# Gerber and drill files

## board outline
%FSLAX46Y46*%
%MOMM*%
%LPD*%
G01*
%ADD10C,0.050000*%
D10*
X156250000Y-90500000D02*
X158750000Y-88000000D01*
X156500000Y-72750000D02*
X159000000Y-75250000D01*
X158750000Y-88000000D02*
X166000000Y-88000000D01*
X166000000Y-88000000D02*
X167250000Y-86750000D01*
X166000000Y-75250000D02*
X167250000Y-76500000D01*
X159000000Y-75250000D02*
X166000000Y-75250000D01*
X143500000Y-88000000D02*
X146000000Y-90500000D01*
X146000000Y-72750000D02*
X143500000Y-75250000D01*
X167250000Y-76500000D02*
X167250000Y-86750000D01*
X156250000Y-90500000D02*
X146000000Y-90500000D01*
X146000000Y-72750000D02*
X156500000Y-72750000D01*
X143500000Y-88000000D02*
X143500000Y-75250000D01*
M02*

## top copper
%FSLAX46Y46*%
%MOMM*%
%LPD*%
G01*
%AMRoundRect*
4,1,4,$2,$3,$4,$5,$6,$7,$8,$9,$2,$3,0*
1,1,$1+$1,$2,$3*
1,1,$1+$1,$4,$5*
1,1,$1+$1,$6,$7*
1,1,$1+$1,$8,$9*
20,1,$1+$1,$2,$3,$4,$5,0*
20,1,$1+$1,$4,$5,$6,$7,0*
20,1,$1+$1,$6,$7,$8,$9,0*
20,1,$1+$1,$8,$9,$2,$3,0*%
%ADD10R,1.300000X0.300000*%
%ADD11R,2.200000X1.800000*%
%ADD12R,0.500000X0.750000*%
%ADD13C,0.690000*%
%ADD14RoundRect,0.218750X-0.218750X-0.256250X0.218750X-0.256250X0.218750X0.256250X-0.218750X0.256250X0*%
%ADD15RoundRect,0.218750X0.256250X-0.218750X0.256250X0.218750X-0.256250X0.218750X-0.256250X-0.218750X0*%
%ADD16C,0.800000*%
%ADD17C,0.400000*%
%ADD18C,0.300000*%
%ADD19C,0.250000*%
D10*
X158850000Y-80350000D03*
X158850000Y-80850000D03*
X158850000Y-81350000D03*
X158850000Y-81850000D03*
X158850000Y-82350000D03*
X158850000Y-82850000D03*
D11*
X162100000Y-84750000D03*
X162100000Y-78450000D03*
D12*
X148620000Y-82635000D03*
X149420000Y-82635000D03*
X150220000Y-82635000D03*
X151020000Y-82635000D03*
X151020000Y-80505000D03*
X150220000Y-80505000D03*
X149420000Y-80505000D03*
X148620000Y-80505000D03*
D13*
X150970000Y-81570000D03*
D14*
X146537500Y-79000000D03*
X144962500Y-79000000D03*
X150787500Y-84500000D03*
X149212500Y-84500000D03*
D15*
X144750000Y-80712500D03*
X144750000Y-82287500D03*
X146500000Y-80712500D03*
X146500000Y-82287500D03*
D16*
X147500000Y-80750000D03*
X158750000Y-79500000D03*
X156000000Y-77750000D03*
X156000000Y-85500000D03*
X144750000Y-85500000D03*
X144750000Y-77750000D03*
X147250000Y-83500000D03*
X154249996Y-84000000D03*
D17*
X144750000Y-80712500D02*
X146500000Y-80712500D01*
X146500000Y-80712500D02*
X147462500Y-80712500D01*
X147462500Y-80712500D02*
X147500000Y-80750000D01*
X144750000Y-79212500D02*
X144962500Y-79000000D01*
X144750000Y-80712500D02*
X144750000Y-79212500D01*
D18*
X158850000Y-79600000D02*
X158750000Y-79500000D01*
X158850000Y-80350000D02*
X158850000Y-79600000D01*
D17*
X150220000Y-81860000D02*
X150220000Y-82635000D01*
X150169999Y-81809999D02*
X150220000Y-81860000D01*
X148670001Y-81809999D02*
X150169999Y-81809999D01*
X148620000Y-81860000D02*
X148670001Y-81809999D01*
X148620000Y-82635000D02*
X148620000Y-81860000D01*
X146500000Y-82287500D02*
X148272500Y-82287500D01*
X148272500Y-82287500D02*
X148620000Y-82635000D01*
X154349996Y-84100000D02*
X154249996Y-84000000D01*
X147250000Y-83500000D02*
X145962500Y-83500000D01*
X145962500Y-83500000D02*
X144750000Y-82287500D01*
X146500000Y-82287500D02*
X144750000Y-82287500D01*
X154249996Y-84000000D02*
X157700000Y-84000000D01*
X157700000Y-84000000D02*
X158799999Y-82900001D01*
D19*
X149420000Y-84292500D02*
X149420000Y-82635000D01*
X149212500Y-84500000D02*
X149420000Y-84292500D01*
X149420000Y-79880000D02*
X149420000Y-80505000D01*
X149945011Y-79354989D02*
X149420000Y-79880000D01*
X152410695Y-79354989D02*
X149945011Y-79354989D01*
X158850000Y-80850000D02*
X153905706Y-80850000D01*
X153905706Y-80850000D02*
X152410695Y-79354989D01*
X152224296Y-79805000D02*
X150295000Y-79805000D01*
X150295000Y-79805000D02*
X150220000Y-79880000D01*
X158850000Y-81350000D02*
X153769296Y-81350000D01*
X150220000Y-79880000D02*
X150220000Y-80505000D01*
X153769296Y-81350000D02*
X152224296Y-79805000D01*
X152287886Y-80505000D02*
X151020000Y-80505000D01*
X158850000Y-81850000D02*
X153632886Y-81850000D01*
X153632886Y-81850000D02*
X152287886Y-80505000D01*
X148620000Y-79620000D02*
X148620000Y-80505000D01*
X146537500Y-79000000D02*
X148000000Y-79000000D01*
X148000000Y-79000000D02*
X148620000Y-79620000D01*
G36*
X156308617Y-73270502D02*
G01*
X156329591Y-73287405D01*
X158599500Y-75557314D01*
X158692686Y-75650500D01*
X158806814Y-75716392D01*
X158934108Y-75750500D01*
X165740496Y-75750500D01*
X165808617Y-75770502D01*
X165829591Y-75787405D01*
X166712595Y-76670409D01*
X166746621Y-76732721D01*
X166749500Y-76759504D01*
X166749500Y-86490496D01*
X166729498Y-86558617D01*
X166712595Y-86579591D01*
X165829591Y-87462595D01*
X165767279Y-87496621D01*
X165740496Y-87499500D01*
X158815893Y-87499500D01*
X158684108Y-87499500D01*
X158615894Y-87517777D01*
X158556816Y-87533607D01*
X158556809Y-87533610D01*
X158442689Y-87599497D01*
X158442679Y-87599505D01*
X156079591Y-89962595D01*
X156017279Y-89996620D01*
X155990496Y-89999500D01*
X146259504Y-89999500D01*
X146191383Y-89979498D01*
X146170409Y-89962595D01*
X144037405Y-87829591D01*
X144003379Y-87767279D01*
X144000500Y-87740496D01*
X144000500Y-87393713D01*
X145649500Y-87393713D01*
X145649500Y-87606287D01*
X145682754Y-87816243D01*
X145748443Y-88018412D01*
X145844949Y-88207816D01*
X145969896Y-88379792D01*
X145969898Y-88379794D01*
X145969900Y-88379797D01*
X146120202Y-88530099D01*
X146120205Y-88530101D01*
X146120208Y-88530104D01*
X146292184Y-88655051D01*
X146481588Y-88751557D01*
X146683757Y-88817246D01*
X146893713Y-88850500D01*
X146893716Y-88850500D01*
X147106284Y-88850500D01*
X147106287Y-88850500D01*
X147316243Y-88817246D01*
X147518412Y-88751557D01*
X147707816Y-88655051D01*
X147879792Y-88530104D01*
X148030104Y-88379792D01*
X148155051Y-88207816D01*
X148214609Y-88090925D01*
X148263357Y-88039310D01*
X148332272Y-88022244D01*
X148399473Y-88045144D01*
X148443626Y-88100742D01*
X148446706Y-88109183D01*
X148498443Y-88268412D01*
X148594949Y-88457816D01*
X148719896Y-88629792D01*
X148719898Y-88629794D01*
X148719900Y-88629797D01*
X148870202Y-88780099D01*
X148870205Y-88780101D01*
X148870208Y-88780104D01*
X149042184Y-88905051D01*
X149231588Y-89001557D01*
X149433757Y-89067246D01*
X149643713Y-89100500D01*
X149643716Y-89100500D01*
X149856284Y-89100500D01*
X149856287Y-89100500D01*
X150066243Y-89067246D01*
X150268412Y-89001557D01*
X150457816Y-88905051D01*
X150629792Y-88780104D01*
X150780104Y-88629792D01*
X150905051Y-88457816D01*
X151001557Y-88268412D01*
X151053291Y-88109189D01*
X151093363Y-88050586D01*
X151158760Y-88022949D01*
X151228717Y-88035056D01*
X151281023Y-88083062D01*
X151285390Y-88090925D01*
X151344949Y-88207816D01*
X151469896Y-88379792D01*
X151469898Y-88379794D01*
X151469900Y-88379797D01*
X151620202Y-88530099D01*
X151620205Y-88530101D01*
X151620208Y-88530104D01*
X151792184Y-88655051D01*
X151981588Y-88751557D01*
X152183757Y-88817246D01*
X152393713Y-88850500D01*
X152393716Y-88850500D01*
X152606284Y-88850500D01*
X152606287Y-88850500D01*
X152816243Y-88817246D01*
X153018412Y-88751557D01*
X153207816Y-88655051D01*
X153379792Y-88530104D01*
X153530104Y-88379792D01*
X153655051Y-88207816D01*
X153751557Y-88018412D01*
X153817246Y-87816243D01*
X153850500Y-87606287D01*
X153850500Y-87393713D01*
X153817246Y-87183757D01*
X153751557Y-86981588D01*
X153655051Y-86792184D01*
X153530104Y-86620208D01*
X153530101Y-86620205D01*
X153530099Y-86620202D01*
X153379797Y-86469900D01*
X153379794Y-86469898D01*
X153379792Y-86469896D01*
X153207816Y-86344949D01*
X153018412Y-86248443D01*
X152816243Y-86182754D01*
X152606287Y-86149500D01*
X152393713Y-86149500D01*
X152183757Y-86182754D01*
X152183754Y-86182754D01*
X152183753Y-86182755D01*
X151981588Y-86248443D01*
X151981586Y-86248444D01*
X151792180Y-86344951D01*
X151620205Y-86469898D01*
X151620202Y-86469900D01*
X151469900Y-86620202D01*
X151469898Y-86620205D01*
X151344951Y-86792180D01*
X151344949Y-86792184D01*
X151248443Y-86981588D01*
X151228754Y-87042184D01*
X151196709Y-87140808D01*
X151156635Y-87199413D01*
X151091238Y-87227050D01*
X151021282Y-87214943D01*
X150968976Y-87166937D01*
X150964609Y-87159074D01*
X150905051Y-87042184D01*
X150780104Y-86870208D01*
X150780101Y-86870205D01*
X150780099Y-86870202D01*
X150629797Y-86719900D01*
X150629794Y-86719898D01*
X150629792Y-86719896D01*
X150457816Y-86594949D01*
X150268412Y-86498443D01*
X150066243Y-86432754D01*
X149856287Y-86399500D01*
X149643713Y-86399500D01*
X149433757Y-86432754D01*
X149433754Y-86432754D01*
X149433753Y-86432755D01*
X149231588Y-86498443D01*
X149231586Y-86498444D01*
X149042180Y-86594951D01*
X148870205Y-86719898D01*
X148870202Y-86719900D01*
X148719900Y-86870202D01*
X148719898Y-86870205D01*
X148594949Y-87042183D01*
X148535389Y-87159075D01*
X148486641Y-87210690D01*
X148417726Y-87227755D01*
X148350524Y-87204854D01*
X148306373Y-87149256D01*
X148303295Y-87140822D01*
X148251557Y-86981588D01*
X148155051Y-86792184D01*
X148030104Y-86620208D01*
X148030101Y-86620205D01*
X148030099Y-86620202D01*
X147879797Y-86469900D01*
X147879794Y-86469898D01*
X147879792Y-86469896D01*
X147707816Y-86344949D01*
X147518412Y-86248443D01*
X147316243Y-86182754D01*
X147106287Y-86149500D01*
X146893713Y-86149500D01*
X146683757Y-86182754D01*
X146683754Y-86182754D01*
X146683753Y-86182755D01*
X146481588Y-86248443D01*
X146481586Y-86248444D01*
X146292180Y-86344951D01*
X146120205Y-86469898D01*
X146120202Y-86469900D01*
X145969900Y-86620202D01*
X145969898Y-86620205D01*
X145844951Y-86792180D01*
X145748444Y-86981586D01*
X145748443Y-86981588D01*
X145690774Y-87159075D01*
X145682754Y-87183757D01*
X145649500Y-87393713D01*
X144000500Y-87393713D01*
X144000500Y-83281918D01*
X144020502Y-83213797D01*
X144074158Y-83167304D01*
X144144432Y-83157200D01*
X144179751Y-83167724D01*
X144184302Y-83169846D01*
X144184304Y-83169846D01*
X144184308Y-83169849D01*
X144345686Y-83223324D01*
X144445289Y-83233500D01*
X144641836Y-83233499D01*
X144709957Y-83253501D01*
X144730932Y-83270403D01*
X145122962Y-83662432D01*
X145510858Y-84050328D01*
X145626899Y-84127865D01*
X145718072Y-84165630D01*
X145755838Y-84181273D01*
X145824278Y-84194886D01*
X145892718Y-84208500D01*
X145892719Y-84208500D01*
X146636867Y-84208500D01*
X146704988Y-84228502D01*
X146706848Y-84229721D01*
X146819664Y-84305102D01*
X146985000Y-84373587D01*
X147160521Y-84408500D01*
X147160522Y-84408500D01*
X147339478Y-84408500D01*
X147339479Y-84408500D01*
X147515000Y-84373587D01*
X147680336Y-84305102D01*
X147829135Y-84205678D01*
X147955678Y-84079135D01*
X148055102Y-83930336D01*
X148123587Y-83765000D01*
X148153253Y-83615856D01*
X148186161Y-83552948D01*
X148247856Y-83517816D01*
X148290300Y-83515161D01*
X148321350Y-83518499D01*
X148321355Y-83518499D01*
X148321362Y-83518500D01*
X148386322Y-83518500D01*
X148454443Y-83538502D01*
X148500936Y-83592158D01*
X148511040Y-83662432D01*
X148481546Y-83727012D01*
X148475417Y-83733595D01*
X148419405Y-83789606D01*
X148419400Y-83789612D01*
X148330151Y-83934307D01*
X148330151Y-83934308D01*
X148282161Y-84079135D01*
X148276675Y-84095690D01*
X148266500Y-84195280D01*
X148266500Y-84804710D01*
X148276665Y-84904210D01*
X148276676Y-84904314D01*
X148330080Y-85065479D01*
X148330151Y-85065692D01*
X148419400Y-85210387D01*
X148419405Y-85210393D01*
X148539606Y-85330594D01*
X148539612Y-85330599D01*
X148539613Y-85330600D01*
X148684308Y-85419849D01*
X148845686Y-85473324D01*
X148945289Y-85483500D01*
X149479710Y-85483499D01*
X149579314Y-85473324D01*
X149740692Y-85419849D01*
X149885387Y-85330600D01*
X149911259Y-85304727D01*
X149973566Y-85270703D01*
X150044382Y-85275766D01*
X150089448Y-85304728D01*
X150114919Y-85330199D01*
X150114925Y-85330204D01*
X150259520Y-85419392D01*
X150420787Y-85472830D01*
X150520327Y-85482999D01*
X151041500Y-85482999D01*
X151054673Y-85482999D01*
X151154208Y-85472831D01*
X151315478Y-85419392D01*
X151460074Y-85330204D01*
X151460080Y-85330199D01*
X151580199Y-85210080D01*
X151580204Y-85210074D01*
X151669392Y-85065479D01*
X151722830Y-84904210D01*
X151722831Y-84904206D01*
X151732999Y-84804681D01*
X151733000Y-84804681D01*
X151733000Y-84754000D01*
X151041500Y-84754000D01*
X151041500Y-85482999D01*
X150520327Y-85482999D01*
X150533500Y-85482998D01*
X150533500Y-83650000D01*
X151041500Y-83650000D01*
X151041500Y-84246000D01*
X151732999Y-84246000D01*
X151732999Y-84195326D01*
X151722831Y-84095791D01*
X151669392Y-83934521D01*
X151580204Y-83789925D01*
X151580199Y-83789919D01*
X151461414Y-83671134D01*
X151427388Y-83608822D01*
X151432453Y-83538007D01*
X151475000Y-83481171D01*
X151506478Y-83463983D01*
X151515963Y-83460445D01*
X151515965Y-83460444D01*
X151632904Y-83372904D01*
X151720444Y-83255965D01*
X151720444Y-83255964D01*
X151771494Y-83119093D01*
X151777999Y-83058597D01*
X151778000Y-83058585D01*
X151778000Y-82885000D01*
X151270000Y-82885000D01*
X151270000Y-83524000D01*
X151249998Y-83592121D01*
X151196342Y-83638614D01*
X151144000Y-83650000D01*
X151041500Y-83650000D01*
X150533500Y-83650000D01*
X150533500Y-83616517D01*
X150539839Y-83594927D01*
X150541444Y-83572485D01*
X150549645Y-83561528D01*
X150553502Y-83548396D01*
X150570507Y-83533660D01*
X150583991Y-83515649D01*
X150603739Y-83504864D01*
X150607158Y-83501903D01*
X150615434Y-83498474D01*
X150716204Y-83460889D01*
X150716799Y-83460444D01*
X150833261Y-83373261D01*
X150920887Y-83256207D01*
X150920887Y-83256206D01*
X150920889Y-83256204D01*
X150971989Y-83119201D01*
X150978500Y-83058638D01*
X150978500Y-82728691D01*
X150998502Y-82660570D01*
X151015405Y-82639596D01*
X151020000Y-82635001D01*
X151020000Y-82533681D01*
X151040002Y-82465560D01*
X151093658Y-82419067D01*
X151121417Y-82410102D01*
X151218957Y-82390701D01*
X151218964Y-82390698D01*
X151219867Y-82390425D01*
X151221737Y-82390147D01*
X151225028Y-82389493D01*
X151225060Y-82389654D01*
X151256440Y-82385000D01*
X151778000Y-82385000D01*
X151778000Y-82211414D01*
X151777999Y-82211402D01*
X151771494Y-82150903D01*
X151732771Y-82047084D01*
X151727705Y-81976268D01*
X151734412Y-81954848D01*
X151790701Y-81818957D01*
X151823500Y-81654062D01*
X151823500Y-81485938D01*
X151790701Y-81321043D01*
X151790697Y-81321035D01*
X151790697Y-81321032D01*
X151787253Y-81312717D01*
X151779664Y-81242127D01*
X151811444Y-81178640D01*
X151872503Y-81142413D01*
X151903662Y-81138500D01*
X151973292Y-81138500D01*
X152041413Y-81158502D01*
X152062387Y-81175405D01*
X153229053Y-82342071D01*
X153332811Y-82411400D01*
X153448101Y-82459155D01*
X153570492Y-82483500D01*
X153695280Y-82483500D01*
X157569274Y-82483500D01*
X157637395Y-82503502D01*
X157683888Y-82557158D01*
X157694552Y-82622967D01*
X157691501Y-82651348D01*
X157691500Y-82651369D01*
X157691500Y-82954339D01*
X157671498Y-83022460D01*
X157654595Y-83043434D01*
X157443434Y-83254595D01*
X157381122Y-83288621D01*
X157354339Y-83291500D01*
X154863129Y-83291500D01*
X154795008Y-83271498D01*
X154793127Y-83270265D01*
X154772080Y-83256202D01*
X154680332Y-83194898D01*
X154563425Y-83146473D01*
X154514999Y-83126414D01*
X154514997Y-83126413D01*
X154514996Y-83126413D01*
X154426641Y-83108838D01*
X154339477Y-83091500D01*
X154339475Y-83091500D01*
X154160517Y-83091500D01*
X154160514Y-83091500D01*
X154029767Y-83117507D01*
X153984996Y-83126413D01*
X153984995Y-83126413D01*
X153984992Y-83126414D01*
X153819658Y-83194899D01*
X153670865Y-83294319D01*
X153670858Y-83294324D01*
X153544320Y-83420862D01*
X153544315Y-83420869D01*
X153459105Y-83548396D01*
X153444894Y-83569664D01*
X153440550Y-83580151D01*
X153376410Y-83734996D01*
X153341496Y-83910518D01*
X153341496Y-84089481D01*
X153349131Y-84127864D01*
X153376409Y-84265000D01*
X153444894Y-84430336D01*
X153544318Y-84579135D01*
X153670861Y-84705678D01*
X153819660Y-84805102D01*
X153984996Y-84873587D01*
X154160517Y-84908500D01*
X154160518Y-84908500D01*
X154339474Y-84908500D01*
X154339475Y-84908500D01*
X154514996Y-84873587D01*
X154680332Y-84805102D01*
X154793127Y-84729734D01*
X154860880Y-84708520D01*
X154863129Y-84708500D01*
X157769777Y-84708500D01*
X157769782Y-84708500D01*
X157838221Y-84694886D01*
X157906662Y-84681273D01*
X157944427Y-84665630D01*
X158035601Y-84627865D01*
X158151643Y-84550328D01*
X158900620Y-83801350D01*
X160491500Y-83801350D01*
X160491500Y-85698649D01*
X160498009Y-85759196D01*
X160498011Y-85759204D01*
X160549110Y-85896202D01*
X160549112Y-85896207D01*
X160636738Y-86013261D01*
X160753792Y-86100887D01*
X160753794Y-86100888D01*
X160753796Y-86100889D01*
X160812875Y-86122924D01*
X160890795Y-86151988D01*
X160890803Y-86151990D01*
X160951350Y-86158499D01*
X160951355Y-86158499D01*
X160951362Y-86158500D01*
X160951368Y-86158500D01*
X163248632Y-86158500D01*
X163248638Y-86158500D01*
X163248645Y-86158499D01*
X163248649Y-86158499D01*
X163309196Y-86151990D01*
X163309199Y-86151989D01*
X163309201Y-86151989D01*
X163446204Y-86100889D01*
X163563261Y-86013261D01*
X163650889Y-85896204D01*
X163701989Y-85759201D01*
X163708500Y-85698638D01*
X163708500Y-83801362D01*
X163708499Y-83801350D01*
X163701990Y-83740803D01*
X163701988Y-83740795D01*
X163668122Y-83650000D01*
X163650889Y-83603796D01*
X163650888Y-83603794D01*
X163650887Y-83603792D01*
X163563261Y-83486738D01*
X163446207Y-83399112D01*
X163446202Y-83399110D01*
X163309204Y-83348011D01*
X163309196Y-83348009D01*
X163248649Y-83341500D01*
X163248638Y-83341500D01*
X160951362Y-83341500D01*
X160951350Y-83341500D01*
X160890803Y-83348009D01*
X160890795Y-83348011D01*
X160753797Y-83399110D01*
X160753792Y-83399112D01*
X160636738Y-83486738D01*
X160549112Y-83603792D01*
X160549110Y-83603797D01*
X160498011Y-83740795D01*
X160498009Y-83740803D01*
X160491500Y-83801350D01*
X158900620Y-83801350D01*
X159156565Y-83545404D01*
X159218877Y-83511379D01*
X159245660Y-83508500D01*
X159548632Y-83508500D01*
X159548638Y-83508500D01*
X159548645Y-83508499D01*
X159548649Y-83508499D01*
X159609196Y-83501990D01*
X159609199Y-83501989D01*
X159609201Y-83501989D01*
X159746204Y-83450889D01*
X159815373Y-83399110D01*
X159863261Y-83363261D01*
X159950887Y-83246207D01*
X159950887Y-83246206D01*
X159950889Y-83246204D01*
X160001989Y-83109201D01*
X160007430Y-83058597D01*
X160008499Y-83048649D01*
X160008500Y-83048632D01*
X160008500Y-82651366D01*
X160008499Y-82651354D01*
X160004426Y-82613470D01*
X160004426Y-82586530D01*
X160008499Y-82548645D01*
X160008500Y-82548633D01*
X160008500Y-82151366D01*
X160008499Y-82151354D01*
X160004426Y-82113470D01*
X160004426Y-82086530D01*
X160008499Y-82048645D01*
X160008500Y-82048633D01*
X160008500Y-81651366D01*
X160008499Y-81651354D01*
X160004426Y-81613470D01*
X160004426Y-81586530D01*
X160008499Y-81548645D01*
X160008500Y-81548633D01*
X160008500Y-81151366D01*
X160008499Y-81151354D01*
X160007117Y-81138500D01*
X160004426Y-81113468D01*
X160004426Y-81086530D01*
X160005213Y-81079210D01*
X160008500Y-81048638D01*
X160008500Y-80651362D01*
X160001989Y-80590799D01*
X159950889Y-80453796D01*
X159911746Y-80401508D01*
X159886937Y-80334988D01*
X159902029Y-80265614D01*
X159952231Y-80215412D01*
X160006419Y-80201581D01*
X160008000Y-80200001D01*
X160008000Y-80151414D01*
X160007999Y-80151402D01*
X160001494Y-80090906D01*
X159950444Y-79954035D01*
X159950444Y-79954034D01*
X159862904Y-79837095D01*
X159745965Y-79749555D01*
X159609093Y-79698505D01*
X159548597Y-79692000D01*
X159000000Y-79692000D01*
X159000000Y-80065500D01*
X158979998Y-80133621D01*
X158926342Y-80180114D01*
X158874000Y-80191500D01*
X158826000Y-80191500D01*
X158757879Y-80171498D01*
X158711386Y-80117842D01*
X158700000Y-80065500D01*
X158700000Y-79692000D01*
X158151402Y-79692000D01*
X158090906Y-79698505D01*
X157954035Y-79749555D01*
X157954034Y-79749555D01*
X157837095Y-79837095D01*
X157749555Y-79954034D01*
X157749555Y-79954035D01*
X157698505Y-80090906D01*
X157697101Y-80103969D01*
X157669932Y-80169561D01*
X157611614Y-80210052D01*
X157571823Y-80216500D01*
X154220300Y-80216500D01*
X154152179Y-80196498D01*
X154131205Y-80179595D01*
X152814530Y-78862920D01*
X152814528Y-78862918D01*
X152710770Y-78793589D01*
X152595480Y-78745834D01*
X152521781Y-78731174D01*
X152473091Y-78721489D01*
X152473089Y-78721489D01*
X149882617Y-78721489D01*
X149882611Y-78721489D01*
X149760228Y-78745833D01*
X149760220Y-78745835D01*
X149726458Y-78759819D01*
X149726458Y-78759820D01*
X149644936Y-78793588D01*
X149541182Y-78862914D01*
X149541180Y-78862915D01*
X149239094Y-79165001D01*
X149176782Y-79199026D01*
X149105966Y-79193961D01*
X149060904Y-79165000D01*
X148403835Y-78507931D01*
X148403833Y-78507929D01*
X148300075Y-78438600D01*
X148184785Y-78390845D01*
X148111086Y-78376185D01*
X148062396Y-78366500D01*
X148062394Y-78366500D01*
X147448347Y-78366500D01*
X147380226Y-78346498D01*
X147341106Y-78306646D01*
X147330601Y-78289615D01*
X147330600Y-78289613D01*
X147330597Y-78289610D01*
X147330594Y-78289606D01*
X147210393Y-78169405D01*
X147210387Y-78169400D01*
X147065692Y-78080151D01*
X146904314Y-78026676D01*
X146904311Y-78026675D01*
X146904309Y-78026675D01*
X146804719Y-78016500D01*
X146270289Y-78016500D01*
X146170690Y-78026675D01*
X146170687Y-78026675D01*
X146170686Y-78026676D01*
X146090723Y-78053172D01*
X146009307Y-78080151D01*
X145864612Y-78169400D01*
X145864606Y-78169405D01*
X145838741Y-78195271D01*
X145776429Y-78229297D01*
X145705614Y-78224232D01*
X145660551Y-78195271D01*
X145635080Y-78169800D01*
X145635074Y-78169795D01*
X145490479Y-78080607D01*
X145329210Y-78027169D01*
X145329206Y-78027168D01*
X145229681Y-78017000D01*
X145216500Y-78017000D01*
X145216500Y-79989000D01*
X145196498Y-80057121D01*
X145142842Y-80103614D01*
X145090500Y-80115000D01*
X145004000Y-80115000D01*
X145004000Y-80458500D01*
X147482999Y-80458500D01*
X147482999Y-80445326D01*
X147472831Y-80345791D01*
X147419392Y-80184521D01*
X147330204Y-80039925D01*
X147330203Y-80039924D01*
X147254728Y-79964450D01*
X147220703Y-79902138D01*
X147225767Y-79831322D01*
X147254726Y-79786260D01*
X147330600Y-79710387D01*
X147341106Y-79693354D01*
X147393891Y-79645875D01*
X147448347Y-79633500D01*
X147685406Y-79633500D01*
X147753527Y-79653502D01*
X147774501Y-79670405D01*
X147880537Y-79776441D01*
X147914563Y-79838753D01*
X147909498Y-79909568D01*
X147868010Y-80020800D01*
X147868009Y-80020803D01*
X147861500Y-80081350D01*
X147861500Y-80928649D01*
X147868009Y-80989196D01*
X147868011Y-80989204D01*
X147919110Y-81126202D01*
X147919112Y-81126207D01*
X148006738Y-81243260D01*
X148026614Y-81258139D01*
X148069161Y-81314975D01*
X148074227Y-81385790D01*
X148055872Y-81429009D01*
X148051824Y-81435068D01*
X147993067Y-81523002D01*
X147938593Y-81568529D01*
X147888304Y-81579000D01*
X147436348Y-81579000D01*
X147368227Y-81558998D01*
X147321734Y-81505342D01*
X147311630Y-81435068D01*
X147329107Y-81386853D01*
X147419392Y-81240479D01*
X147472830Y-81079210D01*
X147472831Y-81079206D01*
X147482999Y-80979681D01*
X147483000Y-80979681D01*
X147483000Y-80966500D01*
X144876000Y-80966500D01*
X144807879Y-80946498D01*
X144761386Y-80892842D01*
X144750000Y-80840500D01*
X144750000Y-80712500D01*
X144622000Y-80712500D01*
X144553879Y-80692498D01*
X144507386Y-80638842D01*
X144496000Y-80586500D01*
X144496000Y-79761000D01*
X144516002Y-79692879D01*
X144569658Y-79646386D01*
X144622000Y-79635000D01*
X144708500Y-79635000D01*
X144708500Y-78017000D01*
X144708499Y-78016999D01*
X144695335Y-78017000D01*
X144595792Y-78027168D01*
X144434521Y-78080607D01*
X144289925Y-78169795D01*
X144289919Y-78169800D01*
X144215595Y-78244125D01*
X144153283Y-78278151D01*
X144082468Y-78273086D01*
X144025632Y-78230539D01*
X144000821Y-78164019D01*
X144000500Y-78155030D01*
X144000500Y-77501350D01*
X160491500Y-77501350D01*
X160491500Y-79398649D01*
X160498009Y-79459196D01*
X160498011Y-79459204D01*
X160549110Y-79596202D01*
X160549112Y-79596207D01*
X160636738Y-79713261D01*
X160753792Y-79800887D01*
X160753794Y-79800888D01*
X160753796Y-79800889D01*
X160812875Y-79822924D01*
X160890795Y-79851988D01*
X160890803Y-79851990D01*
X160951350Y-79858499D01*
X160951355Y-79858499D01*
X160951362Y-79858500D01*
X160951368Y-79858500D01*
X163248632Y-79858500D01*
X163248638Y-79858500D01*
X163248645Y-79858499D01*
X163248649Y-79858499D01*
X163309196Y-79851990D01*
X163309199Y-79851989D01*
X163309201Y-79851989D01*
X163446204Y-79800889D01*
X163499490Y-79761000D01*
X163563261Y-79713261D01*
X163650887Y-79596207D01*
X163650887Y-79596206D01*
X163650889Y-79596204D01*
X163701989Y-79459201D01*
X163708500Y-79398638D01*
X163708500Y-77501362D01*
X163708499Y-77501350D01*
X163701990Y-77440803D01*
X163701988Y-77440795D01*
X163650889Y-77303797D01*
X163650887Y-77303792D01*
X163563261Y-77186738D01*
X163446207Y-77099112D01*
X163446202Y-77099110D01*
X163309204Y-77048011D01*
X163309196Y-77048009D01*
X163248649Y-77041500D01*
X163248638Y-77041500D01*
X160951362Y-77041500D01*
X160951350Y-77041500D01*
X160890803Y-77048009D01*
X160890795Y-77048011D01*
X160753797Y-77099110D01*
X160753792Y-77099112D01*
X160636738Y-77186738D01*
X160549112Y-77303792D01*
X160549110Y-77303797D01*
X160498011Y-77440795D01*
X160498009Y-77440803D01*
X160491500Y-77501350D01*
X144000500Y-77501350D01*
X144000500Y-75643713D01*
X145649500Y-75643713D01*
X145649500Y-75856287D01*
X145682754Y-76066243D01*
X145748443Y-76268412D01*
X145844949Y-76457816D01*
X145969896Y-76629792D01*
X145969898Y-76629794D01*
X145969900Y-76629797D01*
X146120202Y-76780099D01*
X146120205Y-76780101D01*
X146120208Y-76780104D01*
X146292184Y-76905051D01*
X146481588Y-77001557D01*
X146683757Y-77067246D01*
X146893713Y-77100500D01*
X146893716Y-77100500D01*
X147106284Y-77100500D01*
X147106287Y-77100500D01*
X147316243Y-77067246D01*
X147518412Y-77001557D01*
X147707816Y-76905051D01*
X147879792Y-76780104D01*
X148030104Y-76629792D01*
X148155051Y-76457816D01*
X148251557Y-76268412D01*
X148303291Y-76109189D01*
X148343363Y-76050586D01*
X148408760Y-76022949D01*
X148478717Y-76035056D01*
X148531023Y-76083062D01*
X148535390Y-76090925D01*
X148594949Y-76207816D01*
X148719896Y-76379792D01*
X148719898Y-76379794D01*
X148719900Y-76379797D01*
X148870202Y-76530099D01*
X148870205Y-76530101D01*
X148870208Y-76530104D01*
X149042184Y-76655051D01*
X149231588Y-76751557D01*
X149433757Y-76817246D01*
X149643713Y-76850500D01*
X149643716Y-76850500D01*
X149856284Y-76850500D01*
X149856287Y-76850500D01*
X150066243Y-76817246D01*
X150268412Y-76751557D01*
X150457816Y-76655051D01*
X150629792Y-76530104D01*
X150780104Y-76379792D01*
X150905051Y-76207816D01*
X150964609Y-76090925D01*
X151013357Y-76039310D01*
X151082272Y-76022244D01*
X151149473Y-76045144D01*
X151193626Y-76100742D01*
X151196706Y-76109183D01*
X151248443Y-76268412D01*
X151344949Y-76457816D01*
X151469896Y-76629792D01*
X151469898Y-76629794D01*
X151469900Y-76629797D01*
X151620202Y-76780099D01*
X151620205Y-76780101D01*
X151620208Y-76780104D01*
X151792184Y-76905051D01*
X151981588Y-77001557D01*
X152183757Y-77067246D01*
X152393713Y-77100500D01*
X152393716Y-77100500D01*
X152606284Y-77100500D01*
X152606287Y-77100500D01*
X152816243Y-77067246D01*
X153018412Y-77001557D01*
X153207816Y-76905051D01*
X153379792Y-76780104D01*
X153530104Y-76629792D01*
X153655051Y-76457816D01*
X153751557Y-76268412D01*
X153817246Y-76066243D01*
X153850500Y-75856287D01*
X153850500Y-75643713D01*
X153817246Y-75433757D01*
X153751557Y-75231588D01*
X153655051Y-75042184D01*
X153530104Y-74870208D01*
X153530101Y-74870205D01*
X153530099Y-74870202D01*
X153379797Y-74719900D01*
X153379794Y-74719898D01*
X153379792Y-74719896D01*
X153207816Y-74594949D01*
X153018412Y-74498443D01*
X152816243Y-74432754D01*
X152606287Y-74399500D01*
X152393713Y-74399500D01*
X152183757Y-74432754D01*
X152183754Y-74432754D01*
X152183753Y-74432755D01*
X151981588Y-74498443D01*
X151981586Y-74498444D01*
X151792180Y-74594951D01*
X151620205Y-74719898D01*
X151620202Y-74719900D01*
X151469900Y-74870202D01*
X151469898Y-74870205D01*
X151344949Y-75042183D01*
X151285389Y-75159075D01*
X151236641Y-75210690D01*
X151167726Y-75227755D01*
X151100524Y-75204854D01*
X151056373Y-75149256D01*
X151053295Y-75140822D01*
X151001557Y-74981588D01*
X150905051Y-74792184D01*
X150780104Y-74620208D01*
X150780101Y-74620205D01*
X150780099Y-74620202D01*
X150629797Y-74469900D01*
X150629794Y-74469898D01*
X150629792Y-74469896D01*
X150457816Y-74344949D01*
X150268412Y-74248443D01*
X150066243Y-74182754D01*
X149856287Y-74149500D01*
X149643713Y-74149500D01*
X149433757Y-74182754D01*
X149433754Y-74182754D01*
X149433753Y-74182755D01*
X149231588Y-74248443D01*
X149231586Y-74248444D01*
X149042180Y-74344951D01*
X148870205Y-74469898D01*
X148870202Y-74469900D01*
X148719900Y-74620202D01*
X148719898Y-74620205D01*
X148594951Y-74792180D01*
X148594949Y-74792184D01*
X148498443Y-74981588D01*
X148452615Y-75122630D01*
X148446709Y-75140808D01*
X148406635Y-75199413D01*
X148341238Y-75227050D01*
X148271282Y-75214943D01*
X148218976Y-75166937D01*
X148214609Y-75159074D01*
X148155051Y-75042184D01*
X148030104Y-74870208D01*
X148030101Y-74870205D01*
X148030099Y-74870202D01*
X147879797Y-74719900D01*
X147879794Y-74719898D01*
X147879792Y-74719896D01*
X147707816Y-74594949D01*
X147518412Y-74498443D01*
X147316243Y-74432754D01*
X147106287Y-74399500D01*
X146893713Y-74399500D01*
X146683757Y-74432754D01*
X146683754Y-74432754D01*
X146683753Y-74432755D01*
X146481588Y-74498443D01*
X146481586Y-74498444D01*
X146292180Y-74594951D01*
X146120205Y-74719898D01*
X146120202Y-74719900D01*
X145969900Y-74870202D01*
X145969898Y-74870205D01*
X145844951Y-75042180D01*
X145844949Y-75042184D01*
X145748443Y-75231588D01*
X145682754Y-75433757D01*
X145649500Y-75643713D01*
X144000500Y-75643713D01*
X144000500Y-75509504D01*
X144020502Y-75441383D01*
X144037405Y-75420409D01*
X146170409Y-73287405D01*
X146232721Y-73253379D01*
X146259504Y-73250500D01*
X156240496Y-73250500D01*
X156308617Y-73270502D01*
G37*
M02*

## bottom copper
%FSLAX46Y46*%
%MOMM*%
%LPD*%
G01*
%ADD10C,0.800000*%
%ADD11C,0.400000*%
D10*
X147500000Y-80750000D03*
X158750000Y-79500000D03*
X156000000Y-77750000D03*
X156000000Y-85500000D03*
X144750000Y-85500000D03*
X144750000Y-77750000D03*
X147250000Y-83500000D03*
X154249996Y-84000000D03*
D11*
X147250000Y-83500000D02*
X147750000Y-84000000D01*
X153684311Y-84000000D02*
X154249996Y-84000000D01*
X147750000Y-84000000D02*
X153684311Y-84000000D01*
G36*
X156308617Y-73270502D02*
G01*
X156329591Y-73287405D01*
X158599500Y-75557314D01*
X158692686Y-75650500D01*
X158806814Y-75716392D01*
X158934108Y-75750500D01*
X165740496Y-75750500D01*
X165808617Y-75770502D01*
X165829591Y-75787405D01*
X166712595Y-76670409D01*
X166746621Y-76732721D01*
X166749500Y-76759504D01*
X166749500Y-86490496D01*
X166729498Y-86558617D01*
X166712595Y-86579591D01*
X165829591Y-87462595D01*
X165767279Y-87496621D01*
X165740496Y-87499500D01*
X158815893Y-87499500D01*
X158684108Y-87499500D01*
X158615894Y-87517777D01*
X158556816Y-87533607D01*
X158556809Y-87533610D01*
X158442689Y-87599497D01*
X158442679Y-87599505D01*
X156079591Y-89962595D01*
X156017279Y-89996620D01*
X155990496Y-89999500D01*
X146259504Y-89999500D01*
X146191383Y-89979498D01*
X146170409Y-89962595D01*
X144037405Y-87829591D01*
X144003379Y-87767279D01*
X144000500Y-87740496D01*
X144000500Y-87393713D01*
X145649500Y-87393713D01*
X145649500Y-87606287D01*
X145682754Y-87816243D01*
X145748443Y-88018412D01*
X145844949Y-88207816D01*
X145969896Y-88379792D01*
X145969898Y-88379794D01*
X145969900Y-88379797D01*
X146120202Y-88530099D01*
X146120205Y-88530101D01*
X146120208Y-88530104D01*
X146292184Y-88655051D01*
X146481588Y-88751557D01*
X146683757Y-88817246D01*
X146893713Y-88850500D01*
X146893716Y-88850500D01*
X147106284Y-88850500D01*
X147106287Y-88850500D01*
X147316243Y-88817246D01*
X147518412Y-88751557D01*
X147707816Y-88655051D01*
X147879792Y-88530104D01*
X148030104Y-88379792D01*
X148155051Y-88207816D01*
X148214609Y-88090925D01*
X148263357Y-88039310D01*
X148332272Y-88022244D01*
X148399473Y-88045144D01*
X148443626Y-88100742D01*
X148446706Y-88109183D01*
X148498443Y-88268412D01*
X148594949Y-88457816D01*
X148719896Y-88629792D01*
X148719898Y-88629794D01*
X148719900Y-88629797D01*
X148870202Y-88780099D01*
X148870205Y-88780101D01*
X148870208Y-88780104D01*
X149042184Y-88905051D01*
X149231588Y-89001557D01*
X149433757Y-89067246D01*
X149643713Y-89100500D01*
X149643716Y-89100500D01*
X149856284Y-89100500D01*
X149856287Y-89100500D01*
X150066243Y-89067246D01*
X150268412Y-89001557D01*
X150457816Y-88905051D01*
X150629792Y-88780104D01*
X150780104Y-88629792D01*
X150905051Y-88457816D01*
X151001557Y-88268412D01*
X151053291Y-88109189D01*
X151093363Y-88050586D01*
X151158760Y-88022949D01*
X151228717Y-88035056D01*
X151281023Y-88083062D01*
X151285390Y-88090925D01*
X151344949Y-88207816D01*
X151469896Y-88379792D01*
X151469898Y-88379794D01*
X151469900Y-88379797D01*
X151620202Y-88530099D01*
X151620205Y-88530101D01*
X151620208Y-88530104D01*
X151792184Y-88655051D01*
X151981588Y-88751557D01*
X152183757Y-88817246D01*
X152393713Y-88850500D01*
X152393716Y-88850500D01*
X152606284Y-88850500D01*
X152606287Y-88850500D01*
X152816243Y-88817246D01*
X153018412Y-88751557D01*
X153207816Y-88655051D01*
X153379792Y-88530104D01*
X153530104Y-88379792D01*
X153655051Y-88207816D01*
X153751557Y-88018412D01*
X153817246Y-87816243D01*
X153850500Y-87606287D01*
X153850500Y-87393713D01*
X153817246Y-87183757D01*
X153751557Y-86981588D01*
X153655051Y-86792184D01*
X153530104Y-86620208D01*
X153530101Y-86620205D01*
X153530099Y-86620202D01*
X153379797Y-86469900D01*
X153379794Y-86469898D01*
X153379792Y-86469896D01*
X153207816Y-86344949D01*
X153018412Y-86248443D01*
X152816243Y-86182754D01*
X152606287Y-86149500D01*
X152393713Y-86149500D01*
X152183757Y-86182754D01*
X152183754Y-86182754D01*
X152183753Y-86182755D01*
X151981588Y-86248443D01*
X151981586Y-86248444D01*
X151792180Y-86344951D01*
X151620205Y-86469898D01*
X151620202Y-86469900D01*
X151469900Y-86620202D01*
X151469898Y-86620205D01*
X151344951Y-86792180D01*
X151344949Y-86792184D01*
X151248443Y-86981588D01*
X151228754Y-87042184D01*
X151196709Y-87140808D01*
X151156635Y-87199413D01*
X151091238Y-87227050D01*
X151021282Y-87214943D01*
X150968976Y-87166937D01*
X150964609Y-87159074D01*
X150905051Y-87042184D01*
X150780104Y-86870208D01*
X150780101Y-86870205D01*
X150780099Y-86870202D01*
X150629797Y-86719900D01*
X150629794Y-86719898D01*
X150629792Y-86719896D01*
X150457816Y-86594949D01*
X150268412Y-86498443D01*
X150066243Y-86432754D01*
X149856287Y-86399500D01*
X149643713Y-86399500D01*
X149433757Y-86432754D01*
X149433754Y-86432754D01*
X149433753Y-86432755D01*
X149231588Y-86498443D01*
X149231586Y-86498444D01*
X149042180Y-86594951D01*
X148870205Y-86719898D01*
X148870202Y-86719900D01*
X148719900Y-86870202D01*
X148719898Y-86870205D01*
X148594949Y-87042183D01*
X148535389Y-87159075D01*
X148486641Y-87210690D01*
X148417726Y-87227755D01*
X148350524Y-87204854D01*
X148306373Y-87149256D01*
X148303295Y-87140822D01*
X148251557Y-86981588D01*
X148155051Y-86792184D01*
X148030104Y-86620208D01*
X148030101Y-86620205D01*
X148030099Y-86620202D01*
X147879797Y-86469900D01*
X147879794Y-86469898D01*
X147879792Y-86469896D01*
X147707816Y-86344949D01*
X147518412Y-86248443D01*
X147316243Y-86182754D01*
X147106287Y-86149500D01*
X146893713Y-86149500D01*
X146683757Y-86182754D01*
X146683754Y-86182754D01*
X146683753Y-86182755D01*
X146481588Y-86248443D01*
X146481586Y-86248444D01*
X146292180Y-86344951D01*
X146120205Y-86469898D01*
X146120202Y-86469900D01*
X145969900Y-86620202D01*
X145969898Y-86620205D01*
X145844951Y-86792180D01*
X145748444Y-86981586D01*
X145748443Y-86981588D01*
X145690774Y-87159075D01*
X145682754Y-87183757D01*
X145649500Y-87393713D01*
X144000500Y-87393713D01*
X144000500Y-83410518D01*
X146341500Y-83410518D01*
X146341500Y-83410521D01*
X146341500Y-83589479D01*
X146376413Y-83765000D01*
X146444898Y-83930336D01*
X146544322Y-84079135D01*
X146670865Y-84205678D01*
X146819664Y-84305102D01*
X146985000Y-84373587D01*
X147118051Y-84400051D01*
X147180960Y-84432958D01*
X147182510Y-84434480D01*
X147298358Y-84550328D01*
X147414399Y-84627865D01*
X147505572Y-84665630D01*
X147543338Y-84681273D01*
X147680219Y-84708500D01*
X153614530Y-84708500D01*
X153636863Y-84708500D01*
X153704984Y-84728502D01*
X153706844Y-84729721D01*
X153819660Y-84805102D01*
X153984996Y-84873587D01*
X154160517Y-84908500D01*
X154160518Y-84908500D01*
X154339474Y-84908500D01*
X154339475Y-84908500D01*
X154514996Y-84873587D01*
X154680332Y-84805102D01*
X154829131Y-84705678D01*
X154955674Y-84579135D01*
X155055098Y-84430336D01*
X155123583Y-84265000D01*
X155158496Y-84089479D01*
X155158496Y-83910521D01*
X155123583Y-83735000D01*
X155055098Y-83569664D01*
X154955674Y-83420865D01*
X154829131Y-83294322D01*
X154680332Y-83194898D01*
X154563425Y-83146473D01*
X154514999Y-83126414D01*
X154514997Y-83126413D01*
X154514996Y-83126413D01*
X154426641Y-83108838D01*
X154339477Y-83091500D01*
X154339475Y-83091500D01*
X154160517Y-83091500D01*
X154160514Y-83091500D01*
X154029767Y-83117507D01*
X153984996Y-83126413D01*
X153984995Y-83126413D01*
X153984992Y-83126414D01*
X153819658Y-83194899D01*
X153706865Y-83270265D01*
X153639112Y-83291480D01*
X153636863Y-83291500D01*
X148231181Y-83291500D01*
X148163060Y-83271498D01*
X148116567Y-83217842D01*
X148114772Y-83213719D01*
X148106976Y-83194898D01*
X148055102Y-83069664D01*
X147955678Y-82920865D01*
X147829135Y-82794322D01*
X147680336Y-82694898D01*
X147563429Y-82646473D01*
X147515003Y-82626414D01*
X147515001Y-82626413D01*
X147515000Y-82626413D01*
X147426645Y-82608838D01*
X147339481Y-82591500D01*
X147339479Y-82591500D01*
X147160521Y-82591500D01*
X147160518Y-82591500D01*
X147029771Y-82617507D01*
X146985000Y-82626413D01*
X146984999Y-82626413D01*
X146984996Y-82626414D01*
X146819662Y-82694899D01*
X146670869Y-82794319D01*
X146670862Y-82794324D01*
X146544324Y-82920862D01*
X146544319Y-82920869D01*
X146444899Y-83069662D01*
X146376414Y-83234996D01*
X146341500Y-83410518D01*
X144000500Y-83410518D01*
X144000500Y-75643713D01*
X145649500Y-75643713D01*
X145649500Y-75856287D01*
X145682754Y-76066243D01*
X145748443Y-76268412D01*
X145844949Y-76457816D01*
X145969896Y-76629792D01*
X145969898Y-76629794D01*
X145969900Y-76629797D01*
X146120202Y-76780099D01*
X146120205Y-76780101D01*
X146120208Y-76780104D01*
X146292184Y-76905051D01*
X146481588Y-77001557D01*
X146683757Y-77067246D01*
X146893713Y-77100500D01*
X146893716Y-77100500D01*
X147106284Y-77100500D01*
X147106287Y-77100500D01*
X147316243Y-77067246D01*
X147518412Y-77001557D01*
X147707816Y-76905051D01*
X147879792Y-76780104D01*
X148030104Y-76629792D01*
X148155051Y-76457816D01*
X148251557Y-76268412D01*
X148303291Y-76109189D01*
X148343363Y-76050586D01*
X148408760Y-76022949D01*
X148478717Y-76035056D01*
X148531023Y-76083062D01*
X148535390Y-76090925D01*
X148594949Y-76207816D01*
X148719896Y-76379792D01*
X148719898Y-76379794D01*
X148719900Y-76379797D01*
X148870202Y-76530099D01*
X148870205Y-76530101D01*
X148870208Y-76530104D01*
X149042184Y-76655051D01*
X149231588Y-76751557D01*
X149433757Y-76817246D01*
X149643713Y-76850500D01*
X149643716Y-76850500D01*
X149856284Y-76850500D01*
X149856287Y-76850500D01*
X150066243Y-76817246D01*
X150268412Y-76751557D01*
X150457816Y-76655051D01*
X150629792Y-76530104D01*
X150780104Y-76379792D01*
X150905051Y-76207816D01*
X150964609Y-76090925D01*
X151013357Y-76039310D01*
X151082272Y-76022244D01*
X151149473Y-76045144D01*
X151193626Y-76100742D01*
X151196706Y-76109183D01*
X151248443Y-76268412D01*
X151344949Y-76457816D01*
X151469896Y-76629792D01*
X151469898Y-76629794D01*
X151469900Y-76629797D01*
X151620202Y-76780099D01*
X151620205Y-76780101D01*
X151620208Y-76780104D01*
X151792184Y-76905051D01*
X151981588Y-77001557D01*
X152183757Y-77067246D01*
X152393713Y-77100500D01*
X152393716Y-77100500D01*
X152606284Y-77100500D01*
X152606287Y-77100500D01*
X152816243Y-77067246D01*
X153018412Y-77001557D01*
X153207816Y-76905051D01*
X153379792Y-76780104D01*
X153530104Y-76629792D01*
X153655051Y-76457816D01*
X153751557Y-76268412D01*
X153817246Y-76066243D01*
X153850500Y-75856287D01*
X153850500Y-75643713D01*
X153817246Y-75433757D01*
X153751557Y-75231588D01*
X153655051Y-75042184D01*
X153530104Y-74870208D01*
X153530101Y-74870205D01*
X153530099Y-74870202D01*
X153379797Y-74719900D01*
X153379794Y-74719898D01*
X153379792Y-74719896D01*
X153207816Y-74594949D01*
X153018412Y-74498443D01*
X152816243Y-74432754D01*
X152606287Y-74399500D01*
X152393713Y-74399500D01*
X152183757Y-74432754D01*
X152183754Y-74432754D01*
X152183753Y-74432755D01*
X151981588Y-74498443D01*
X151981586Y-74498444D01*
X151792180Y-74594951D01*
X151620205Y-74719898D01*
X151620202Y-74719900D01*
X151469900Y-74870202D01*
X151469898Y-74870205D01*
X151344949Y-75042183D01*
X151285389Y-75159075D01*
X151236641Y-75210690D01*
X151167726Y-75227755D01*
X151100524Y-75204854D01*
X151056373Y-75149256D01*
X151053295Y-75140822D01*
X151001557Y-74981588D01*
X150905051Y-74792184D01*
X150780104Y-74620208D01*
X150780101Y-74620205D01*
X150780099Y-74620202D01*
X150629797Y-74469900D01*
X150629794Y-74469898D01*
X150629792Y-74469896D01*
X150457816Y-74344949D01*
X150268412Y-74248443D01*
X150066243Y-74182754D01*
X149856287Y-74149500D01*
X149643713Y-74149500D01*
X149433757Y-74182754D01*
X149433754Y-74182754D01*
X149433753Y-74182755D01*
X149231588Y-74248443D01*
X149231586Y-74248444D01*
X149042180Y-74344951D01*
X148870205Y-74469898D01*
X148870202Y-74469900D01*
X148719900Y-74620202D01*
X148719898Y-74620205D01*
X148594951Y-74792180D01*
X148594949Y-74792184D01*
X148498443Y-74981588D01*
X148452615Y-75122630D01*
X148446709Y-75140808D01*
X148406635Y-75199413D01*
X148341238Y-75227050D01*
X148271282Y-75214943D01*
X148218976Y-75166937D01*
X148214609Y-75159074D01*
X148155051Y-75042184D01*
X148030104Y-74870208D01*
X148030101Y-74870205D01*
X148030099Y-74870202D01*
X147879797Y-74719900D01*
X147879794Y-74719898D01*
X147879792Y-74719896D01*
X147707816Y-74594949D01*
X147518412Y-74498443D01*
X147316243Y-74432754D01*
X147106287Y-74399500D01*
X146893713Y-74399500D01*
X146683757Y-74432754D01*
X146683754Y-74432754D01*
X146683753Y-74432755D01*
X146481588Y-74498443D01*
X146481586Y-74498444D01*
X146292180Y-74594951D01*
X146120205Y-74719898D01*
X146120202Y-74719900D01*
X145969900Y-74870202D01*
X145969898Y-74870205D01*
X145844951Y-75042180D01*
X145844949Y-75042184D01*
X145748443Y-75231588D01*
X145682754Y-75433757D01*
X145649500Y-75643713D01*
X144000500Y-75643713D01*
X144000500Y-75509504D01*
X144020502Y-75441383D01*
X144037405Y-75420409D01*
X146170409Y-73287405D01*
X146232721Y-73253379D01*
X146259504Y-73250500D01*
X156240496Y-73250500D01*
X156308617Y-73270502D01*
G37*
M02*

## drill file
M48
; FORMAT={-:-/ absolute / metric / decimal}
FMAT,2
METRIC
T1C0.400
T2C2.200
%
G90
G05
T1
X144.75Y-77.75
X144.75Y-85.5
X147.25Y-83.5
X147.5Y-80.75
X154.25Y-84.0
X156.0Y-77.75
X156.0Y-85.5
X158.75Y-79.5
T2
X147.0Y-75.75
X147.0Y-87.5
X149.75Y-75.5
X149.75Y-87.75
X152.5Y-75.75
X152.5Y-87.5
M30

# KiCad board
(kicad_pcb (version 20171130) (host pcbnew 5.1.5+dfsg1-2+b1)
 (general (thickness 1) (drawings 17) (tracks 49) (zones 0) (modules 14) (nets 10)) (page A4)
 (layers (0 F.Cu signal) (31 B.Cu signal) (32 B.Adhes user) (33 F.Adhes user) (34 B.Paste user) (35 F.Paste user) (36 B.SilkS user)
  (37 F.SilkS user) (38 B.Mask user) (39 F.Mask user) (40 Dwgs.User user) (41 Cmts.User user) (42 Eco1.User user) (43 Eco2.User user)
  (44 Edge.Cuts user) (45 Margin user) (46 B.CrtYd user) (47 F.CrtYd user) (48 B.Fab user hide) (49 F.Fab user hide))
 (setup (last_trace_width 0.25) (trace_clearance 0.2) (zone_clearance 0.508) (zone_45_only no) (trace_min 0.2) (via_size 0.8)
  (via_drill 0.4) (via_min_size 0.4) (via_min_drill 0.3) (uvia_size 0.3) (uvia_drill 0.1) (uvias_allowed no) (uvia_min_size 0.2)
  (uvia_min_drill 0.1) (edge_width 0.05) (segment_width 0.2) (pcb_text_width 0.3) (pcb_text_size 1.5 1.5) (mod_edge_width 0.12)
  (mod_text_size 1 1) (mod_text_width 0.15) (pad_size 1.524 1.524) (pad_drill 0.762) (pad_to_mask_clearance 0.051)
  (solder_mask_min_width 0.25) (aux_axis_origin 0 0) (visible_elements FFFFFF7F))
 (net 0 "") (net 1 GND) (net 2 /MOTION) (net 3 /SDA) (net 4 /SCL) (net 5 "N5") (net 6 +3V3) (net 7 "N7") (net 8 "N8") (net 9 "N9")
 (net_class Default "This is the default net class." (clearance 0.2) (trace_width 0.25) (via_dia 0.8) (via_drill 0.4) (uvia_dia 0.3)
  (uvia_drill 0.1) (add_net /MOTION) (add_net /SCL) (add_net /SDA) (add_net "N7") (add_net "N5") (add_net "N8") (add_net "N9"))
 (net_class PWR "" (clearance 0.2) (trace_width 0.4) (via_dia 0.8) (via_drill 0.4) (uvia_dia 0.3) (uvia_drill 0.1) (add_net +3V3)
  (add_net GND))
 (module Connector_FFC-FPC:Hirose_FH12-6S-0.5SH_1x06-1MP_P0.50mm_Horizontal (layer F.Cu) (at 160.7 81.6 90)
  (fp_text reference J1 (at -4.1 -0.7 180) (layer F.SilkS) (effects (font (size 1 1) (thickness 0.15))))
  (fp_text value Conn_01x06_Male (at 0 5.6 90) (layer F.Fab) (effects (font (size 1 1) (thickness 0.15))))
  (pad 6 smd rect (at 1.25 -1.85 90) (size 0.3 1.3) (layers F.Cu F.Paste F.Mask) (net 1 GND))
  (pad 5 smd rect (at 0.75 -1.85 90) (size 0.3 1.3) (layers F.Cu F.Paste F.Mask) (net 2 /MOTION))
  (pad 4 smd rect (at 0.25 -1.85 90) (size 0.3 1.3) (layers F.Cu F.Paste F.Mask) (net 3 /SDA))
  (pad 3 smd rect (at -0.25 -1.85 90) (size 0.3 1.3) (layers F.Cu F.Paste F.Mask) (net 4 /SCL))
  (pad 2 smd rect (at -0.75 -1.85 90) (size 0.3 1.3) (layers F.Cu F.Paste F.Mask) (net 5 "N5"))
  (pad 1 smd rect (at -1.25 -1.85 90) (size 0.3 1.3) (layers F.Cu F.Paste F.Mask) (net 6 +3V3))
  (pad MP smd rect (at -3.15 1.4 90) (size 1.8 2.2) (layers F.Cu F.Paste F.Mask))
  (pad MP smd rect (at 3.15 1.4 90) (size 1.8 2.2) (layers F.Cu F.Paste F.Mask)))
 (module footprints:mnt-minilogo (layer F.Cu) (at 156.2 81.5 90)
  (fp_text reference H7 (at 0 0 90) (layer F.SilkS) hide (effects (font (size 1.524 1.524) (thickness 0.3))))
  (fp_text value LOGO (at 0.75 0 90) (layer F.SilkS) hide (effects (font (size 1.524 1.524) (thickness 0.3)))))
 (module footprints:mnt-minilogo (layer B.Cu) (at 162 81.75 270)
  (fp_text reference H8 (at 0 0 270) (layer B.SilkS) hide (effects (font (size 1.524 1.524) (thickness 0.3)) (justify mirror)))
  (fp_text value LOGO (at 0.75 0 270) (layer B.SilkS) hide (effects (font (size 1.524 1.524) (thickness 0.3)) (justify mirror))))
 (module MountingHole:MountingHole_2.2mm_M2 (layer F.Cu) (at 147 87.5)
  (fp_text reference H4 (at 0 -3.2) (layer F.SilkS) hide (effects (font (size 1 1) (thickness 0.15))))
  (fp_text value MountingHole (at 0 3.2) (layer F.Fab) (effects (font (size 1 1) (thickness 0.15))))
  (pad 1 np_thru_hole circle (at 0 0) (size 2.2 2.2) (drill 2.2) (layers *.Cu *.Mask)))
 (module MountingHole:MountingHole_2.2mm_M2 (layer F.Cu) (at 152.5 87.5)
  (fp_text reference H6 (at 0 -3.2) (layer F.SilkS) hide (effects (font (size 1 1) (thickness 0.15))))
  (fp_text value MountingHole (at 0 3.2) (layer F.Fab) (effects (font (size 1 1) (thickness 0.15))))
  (pad 1 np_thru_hole circle (at 0 0) (size 2.2 2.2) (drill 2.2) (layers *.Cu *.Mask)))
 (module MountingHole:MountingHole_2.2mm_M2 (layer F.Cu) (at 147 75.75)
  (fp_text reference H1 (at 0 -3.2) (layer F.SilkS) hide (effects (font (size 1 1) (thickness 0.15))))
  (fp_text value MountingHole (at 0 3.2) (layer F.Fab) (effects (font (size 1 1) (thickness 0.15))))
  (pad 1 np_thru_hole circle (at 0 0) (size 2.2 2.2) (drill 2.2) (layers *.Cu *.Mask)))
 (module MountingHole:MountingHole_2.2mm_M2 (layer F.Cu) (at 152.5 75.75)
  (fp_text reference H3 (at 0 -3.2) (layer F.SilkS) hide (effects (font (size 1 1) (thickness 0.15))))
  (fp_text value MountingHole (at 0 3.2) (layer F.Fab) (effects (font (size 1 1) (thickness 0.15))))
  (pad 1 np_thru_hole circle (at 0 0) (size 2.2 2.2) (drill 2.2) (layers *.Cu *.Mask)))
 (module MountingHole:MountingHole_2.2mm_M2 (layer F.Cu) (at 149.75 87.75)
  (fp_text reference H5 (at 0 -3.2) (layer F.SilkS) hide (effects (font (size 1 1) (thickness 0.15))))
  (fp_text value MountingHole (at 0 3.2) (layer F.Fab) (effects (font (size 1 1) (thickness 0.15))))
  (pad 1 np_thru_hole circle (at 0 0) (size 2.2 2.2) (drill 2.2) (layers *.Cu *.Mask)))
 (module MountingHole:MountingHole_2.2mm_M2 (layer F.Cu) (at 149.75 75.5)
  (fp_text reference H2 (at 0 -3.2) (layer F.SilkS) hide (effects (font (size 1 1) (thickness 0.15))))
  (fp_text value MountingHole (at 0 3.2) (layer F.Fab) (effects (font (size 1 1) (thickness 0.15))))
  (pad 1 np_thru_hole circle (at 0 0) (size 2.2 2.2) (drill 2.2) (layers *.Cu *.Mask)))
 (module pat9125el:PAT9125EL (layer F.Cu) (at 149.82 81.57)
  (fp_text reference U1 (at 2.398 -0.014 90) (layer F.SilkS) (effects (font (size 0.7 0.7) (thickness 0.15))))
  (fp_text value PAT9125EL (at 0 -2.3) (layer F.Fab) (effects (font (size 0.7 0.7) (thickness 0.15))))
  (pad 1 smd rect (at -1.2 1.065) (size 0.5 0.75) (layers F.Cu F.Paste F.Mask) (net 6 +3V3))
  (pad 2 smd rect (at -0.4 1.065) (size 0.5 0.75) (layers F.Cu F.Paste F.Mask) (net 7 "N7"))
  (pad 3 smd rect (at 0.4 1.065) (size 0.5 0.75) (layers F.Cu F.Paste F.Mask) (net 6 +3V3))
  (pad 4 smd rect (at 1.2 1.065) (size 0.5 0.75) (layers F.Cu F.Paste F.Mask) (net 1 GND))
  (pad 5 smd rect (at 1.2 -1.065) (size 0.5 0.75) (layers F.Cu F.Paste F.Mask) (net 4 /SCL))
  (pad 6 smd rect (at 0.4 -1.065) (size 0.5 0.75) (layers F.Cu F.Paste F.Mask) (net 3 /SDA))
  (pad 7 smd rect (at -0.4 -1.065) (size 0.5 0.75) (layers F.Cu F.Paste F.Mask) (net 2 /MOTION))
  (pad 8 smd rect (at -1.2 -1.065) (size 0.5 0.75) (layers F.Cu F.Paste F.Mask) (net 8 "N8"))
  (pad 9 smd circle (at 1.15 0) (size 0.69 0.69) (layers F.Cu F.Paste F.Mask) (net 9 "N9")))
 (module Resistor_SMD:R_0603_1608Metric (layer F.Cu) (at 145.75 79)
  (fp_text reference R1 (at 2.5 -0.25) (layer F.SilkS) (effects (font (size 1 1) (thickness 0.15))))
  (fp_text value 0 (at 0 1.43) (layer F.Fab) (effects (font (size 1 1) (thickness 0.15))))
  (pad 2 smd roundrect (at 0.7875 0) (size 0.875 0.95) (layers F.Cu F.Paste F.Mask) (roundrect_rratio 0.25) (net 8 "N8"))
  (pad 1 smd roundrect (at -0.7875 0) (size 0.875 0.95) (layers F.Cu F.Paste F.Mask) (roundrect_rratio 0.25) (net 1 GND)))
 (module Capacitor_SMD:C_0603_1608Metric (layer F.Cu) (at 150 84.5)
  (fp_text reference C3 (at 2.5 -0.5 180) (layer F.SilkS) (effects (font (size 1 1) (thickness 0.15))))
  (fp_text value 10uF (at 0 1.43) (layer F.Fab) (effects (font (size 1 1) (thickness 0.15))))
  (pad 2 smd roundrect (at 0.7875 0) (size 0.875 0.95) (layers F.Cu F.Paste F.Mask) (roundrect_rratio 0.25) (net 1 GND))
  (pad 1 smd roundrect (at -0.7875 0) (size 0.875 0.95) (layers F.Cu F.Paste F.Mask) (roundrect_rratio 0.25) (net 7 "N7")))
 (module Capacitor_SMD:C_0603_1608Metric (layer F.Cu) (at 144.75 81.5 90)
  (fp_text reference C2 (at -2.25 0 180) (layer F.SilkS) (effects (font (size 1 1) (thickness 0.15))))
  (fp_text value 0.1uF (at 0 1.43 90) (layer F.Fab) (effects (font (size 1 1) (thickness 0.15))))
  (pad 2 smd roundrect (at 0.7875 0 90) (size 0.875 0.95) (layers F.Cu F.Paste F.Mask) (roundrect_rratio 0.25) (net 1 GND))
  (pad 1 smd roundrect (at -0.7875 0 90) (size 0.875 0.95) (layers F.Cu F.Paste F.Mask) (roundrect_rratio 0.25) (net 6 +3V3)))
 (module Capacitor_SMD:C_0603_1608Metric (layer F.Cu) (at 146.5 81.5 90)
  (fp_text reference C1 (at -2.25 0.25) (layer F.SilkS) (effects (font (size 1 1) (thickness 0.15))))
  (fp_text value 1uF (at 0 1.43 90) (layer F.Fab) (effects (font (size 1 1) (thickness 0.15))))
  (pad 2 smd roundrect (at 0.7875 0 90) (size 0.875 0.95) (layers F.Cu F.Paste F.Mask) (roundrect_rratio 0.25) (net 1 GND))
  (pad 1 smd roundrect (at -0.7875 0 90) (size 0.875 0.95) (layers F.Cu F.Paste F.Mask) (roundrect_rratio 0.25) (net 6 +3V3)))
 (gr_line (start 156.25 90.5) (end 158.75 88) (layer Edge.Cuts) (width 0.05))
 (gr_line (start 156.5 72.75) (end 159 75.25) (layer Edge.Cuts) (width 0.05))
 (gr_line (start 158.75 88) (end 166 88) (layer Edge.Cuts) (width 0.05))
 (gr_line (start 166 88) (end 167.25 86.75) (layer Edge.Cuts) (width 0.05))
 (gr_line (start 166 75.25) (end 167.25 76.5) (layer Edge.Cuts) (width 0.05))
 (gr_line (start 159 75.25) (end 166 75.25) (layer Edge.Cuts) (width 0.05))
 (gr_line (start 143.5 88) (end 146 90.5) (layer Edge.Cuts) (width 0.05))
 (gr_line (start 146 72.75) (end 143.5 75.25) (layer Edge.Cuts) (width 0.05))
 (gr_line (start 167.25 76.5) (end 167.25 86.75) (layer Edge.Cuts) (width 0.05))
 (gr_line (start 156.25 90.5) (end 146 90.5) (layer Edge.Cuts) (width 0.05))
 (gr_line (start 146 72.75) (end 156.5 72.75) (layer Edge.Cuts) (width 0.05))
 (gr_line (start 143.5 88) (end 143.5 75.25) (layer Edge.Cuts) (width 0.05))
 (segment (start 144.75 80.7125) (end 146.5 80.7125) (width 0.4) (layer F.Cu) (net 1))
 (segment (start 146.5 80.7125) (end 147.4625 80.7125) (width 0.4) (layer F.Cu) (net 1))
 (via (at 147.5 80.75) (size 0.8) (drill 0.4) (layers F.Cu B.Cu) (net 1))
 (segment (start 147.4625 80.7125) (end 147.5 80.75) (width 0.4) (layer F.Cu) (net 1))
 (segment (start 144.75 79.2125) (end 144.9625 79) (width 0.4) (layer F.Cu) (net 1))
 (segment (start 144.75 80.7125) (end 144.75 79.2125) (width 0.4) (layer F.Cu) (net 1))
 (via (at 158.75 79.5) (size 0.8) (drill 0.4) (layers F.Cu B.Cu) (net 1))
 (segment (start 158.85 79.6) (end 158.75 79.5) (width 0.3) (layer F.Cu) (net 1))
 (segment (start 158.85 80.35) (end 158.85 79.6) (width 0.3) (layer F.Cu) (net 1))
 (via (at 156 77.75) (size 0.8) (drill 0.4) (layers F.Cu B.Cu) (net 1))
 (via (at 156 85.5) (size 0.8) (drill 0.4) (layers F.Cu B.Cu) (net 1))
 (via (at 144.75 85.5) (size 0.8) (drill 0.4) (layers F.Cu B.Cu) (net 1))
 (via (at 144.75 77.75) (size 0.8) (drill 0.4) (layers F.Cu B.Cu) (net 1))
 (segment (start 150.22 81.86) (end 150.22 82.635) (width 0.4) (layer F.Cu) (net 6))
 (segment (start 150.169999 81.809999) (end 150.22 81.86) (width 0.4) (layer F.Cu) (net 6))
 (segment (start 148.670001 81.809999) (end 150.169999 81.809999) (width 0.4) (layer F.Cu) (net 6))
 (segment (start 148.62 81.86) (end 148.670001 81.809999) (width 0.4) (layer F.Cu) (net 6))
 (segment (start 148.62 82.635) (end 148.62 81.86) (width 0.4) (layer F.Cu) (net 6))
 (segment (start 146.5 82.2875) (end 148.2725 82.2875) (width 0.4) (layer F.Cu) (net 6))
 (segment (start 148.2725 82.2875) (end 148.62 82.635) (width 0.4) (layer F.Cu) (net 6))
 (via (at 147.25 83.5) (size 0.8) (drill 0.4) (layers F.Cu B.Cu) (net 6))
 (segment (start 147.25 83.5) (end 147.75 84) (width 0.4) (layer B.Cu) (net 6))
 (segment (start 153.684311 84) (end 154.249996 84) (width 0.4) (layer B.Cu) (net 6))
 (segment (start 154.349996 84.1) (end 154.249996 84) (width 0.4) (layer F.Cu) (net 6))
 (segment (start 147.75 84) (end 153.684311 84) (width 0.4) (layer B.Cu) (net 6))
 (via (at 154.249996 84) (size 0.8) (drill 0.4) (layers F.Cu B.Cu) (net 6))
 (segment (start 147.25 83.5) (end 145.9625 83.5) (width 0.4) (layer F.Cu) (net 6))
 (segment (start 145.9625 83.5) (end 144.75 82.2875) (width 0.4) (layer F.Cu) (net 6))
 (segment (start 146.5 82.2875) (end 144.75 82.2875) (width 0.4) (layer F.Cu) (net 6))
 (segment (start 154.249996 84) (end 157.7 84) (width 0.4) (layer F.Cu) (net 6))
 (segment (start 157.7 84) (end 158.799999 82.900001) (width 0.4) (layer F.Cu) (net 6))
 (segment (start 149.42 84.2925) (end 149.42 82.635) (width 0.25) (layer F.Cu) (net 7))
 (segment (start 149.2125 84.5) (end 149.42 84.2925) (width 0.25) (layer F.Cu) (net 7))
 (segment (start 149.42 79.88) (end 149.42 80.505) (width 0.25) (layer F.Cu) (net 2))
 (segment (start 149.945011 79.354989) (end 149.42 79.88) (width 0.25) (layer F.Cu) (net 2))
 (segment (start 152.410695 79.354989) (end 149.945011 79.354989) (width 0.25) (layer F.Cu) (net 2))
 (segment (start 158.85 80.85) (end 153.905706 80.85) (width 0.25) (layer F.Cu) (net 2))
 (segment (start 153.905706 80.85) (end 152.410695 79.354989) (width 0.25) (layer F.Cu) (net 2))
 (segment (start 152.224296 79.805) (end 150.295 79.805) (width 0.25) (layer F.Cu) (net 3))
 (segment (start 150.295 79.805) (end 150.22 79.88) (width 0.25) (layer F.Cu) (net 3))
 (segment (start 158.85 81.35) (end 153.769296 81.35) (width 0.25) (layer F.Cu) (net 3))
 (segment (start 150.22 79.88) (end 150.22 80.505) (width 0.25) (layer F.Cu) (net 3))
 (segment (start 153.769296 81.35) (end 152.224296 79.805) (width 0.25) (layer F.Cu) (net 3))
 (segment (start 152.287886 80.505) (end 151.02 80.505) (width 0.25) (layer F.Cu) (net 4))
 (segment (start 158.85 81.85) (end 153.632886 81.85) (width 0.25) (layer F.Cu) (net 4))
 (segment (start 153.632886 81.85) (end 152.287886 80.505) (width 0.25) (layer F.Cu) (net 4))
 (segment (start 148.62 79.62) (end 148.62 80.505) (width 0.25) (layer F.Cu) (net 8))
 (segment (start 146.5375 79) (end 148 79) (width 0.25) (layer F.Cu) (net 8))
 (segment (start 148 79) (end 148.62 79.62) (width 0.25) (layer F.Cu) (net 8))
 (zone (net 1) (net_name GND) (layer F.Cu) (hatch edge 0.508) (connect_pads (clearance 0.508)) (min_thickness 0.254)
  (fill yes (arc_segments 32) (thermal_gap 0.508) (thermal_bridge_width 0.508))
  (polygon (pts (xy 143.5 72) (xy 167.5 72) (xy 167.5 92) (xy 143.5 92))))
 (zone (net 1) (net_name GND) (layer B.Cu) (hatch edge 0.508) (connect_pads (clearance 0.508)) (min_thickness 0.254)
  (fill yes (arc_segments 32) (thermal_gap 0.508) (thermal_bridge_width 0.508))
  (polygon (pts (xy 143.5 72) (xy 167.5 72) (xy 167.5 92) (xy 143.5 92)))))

